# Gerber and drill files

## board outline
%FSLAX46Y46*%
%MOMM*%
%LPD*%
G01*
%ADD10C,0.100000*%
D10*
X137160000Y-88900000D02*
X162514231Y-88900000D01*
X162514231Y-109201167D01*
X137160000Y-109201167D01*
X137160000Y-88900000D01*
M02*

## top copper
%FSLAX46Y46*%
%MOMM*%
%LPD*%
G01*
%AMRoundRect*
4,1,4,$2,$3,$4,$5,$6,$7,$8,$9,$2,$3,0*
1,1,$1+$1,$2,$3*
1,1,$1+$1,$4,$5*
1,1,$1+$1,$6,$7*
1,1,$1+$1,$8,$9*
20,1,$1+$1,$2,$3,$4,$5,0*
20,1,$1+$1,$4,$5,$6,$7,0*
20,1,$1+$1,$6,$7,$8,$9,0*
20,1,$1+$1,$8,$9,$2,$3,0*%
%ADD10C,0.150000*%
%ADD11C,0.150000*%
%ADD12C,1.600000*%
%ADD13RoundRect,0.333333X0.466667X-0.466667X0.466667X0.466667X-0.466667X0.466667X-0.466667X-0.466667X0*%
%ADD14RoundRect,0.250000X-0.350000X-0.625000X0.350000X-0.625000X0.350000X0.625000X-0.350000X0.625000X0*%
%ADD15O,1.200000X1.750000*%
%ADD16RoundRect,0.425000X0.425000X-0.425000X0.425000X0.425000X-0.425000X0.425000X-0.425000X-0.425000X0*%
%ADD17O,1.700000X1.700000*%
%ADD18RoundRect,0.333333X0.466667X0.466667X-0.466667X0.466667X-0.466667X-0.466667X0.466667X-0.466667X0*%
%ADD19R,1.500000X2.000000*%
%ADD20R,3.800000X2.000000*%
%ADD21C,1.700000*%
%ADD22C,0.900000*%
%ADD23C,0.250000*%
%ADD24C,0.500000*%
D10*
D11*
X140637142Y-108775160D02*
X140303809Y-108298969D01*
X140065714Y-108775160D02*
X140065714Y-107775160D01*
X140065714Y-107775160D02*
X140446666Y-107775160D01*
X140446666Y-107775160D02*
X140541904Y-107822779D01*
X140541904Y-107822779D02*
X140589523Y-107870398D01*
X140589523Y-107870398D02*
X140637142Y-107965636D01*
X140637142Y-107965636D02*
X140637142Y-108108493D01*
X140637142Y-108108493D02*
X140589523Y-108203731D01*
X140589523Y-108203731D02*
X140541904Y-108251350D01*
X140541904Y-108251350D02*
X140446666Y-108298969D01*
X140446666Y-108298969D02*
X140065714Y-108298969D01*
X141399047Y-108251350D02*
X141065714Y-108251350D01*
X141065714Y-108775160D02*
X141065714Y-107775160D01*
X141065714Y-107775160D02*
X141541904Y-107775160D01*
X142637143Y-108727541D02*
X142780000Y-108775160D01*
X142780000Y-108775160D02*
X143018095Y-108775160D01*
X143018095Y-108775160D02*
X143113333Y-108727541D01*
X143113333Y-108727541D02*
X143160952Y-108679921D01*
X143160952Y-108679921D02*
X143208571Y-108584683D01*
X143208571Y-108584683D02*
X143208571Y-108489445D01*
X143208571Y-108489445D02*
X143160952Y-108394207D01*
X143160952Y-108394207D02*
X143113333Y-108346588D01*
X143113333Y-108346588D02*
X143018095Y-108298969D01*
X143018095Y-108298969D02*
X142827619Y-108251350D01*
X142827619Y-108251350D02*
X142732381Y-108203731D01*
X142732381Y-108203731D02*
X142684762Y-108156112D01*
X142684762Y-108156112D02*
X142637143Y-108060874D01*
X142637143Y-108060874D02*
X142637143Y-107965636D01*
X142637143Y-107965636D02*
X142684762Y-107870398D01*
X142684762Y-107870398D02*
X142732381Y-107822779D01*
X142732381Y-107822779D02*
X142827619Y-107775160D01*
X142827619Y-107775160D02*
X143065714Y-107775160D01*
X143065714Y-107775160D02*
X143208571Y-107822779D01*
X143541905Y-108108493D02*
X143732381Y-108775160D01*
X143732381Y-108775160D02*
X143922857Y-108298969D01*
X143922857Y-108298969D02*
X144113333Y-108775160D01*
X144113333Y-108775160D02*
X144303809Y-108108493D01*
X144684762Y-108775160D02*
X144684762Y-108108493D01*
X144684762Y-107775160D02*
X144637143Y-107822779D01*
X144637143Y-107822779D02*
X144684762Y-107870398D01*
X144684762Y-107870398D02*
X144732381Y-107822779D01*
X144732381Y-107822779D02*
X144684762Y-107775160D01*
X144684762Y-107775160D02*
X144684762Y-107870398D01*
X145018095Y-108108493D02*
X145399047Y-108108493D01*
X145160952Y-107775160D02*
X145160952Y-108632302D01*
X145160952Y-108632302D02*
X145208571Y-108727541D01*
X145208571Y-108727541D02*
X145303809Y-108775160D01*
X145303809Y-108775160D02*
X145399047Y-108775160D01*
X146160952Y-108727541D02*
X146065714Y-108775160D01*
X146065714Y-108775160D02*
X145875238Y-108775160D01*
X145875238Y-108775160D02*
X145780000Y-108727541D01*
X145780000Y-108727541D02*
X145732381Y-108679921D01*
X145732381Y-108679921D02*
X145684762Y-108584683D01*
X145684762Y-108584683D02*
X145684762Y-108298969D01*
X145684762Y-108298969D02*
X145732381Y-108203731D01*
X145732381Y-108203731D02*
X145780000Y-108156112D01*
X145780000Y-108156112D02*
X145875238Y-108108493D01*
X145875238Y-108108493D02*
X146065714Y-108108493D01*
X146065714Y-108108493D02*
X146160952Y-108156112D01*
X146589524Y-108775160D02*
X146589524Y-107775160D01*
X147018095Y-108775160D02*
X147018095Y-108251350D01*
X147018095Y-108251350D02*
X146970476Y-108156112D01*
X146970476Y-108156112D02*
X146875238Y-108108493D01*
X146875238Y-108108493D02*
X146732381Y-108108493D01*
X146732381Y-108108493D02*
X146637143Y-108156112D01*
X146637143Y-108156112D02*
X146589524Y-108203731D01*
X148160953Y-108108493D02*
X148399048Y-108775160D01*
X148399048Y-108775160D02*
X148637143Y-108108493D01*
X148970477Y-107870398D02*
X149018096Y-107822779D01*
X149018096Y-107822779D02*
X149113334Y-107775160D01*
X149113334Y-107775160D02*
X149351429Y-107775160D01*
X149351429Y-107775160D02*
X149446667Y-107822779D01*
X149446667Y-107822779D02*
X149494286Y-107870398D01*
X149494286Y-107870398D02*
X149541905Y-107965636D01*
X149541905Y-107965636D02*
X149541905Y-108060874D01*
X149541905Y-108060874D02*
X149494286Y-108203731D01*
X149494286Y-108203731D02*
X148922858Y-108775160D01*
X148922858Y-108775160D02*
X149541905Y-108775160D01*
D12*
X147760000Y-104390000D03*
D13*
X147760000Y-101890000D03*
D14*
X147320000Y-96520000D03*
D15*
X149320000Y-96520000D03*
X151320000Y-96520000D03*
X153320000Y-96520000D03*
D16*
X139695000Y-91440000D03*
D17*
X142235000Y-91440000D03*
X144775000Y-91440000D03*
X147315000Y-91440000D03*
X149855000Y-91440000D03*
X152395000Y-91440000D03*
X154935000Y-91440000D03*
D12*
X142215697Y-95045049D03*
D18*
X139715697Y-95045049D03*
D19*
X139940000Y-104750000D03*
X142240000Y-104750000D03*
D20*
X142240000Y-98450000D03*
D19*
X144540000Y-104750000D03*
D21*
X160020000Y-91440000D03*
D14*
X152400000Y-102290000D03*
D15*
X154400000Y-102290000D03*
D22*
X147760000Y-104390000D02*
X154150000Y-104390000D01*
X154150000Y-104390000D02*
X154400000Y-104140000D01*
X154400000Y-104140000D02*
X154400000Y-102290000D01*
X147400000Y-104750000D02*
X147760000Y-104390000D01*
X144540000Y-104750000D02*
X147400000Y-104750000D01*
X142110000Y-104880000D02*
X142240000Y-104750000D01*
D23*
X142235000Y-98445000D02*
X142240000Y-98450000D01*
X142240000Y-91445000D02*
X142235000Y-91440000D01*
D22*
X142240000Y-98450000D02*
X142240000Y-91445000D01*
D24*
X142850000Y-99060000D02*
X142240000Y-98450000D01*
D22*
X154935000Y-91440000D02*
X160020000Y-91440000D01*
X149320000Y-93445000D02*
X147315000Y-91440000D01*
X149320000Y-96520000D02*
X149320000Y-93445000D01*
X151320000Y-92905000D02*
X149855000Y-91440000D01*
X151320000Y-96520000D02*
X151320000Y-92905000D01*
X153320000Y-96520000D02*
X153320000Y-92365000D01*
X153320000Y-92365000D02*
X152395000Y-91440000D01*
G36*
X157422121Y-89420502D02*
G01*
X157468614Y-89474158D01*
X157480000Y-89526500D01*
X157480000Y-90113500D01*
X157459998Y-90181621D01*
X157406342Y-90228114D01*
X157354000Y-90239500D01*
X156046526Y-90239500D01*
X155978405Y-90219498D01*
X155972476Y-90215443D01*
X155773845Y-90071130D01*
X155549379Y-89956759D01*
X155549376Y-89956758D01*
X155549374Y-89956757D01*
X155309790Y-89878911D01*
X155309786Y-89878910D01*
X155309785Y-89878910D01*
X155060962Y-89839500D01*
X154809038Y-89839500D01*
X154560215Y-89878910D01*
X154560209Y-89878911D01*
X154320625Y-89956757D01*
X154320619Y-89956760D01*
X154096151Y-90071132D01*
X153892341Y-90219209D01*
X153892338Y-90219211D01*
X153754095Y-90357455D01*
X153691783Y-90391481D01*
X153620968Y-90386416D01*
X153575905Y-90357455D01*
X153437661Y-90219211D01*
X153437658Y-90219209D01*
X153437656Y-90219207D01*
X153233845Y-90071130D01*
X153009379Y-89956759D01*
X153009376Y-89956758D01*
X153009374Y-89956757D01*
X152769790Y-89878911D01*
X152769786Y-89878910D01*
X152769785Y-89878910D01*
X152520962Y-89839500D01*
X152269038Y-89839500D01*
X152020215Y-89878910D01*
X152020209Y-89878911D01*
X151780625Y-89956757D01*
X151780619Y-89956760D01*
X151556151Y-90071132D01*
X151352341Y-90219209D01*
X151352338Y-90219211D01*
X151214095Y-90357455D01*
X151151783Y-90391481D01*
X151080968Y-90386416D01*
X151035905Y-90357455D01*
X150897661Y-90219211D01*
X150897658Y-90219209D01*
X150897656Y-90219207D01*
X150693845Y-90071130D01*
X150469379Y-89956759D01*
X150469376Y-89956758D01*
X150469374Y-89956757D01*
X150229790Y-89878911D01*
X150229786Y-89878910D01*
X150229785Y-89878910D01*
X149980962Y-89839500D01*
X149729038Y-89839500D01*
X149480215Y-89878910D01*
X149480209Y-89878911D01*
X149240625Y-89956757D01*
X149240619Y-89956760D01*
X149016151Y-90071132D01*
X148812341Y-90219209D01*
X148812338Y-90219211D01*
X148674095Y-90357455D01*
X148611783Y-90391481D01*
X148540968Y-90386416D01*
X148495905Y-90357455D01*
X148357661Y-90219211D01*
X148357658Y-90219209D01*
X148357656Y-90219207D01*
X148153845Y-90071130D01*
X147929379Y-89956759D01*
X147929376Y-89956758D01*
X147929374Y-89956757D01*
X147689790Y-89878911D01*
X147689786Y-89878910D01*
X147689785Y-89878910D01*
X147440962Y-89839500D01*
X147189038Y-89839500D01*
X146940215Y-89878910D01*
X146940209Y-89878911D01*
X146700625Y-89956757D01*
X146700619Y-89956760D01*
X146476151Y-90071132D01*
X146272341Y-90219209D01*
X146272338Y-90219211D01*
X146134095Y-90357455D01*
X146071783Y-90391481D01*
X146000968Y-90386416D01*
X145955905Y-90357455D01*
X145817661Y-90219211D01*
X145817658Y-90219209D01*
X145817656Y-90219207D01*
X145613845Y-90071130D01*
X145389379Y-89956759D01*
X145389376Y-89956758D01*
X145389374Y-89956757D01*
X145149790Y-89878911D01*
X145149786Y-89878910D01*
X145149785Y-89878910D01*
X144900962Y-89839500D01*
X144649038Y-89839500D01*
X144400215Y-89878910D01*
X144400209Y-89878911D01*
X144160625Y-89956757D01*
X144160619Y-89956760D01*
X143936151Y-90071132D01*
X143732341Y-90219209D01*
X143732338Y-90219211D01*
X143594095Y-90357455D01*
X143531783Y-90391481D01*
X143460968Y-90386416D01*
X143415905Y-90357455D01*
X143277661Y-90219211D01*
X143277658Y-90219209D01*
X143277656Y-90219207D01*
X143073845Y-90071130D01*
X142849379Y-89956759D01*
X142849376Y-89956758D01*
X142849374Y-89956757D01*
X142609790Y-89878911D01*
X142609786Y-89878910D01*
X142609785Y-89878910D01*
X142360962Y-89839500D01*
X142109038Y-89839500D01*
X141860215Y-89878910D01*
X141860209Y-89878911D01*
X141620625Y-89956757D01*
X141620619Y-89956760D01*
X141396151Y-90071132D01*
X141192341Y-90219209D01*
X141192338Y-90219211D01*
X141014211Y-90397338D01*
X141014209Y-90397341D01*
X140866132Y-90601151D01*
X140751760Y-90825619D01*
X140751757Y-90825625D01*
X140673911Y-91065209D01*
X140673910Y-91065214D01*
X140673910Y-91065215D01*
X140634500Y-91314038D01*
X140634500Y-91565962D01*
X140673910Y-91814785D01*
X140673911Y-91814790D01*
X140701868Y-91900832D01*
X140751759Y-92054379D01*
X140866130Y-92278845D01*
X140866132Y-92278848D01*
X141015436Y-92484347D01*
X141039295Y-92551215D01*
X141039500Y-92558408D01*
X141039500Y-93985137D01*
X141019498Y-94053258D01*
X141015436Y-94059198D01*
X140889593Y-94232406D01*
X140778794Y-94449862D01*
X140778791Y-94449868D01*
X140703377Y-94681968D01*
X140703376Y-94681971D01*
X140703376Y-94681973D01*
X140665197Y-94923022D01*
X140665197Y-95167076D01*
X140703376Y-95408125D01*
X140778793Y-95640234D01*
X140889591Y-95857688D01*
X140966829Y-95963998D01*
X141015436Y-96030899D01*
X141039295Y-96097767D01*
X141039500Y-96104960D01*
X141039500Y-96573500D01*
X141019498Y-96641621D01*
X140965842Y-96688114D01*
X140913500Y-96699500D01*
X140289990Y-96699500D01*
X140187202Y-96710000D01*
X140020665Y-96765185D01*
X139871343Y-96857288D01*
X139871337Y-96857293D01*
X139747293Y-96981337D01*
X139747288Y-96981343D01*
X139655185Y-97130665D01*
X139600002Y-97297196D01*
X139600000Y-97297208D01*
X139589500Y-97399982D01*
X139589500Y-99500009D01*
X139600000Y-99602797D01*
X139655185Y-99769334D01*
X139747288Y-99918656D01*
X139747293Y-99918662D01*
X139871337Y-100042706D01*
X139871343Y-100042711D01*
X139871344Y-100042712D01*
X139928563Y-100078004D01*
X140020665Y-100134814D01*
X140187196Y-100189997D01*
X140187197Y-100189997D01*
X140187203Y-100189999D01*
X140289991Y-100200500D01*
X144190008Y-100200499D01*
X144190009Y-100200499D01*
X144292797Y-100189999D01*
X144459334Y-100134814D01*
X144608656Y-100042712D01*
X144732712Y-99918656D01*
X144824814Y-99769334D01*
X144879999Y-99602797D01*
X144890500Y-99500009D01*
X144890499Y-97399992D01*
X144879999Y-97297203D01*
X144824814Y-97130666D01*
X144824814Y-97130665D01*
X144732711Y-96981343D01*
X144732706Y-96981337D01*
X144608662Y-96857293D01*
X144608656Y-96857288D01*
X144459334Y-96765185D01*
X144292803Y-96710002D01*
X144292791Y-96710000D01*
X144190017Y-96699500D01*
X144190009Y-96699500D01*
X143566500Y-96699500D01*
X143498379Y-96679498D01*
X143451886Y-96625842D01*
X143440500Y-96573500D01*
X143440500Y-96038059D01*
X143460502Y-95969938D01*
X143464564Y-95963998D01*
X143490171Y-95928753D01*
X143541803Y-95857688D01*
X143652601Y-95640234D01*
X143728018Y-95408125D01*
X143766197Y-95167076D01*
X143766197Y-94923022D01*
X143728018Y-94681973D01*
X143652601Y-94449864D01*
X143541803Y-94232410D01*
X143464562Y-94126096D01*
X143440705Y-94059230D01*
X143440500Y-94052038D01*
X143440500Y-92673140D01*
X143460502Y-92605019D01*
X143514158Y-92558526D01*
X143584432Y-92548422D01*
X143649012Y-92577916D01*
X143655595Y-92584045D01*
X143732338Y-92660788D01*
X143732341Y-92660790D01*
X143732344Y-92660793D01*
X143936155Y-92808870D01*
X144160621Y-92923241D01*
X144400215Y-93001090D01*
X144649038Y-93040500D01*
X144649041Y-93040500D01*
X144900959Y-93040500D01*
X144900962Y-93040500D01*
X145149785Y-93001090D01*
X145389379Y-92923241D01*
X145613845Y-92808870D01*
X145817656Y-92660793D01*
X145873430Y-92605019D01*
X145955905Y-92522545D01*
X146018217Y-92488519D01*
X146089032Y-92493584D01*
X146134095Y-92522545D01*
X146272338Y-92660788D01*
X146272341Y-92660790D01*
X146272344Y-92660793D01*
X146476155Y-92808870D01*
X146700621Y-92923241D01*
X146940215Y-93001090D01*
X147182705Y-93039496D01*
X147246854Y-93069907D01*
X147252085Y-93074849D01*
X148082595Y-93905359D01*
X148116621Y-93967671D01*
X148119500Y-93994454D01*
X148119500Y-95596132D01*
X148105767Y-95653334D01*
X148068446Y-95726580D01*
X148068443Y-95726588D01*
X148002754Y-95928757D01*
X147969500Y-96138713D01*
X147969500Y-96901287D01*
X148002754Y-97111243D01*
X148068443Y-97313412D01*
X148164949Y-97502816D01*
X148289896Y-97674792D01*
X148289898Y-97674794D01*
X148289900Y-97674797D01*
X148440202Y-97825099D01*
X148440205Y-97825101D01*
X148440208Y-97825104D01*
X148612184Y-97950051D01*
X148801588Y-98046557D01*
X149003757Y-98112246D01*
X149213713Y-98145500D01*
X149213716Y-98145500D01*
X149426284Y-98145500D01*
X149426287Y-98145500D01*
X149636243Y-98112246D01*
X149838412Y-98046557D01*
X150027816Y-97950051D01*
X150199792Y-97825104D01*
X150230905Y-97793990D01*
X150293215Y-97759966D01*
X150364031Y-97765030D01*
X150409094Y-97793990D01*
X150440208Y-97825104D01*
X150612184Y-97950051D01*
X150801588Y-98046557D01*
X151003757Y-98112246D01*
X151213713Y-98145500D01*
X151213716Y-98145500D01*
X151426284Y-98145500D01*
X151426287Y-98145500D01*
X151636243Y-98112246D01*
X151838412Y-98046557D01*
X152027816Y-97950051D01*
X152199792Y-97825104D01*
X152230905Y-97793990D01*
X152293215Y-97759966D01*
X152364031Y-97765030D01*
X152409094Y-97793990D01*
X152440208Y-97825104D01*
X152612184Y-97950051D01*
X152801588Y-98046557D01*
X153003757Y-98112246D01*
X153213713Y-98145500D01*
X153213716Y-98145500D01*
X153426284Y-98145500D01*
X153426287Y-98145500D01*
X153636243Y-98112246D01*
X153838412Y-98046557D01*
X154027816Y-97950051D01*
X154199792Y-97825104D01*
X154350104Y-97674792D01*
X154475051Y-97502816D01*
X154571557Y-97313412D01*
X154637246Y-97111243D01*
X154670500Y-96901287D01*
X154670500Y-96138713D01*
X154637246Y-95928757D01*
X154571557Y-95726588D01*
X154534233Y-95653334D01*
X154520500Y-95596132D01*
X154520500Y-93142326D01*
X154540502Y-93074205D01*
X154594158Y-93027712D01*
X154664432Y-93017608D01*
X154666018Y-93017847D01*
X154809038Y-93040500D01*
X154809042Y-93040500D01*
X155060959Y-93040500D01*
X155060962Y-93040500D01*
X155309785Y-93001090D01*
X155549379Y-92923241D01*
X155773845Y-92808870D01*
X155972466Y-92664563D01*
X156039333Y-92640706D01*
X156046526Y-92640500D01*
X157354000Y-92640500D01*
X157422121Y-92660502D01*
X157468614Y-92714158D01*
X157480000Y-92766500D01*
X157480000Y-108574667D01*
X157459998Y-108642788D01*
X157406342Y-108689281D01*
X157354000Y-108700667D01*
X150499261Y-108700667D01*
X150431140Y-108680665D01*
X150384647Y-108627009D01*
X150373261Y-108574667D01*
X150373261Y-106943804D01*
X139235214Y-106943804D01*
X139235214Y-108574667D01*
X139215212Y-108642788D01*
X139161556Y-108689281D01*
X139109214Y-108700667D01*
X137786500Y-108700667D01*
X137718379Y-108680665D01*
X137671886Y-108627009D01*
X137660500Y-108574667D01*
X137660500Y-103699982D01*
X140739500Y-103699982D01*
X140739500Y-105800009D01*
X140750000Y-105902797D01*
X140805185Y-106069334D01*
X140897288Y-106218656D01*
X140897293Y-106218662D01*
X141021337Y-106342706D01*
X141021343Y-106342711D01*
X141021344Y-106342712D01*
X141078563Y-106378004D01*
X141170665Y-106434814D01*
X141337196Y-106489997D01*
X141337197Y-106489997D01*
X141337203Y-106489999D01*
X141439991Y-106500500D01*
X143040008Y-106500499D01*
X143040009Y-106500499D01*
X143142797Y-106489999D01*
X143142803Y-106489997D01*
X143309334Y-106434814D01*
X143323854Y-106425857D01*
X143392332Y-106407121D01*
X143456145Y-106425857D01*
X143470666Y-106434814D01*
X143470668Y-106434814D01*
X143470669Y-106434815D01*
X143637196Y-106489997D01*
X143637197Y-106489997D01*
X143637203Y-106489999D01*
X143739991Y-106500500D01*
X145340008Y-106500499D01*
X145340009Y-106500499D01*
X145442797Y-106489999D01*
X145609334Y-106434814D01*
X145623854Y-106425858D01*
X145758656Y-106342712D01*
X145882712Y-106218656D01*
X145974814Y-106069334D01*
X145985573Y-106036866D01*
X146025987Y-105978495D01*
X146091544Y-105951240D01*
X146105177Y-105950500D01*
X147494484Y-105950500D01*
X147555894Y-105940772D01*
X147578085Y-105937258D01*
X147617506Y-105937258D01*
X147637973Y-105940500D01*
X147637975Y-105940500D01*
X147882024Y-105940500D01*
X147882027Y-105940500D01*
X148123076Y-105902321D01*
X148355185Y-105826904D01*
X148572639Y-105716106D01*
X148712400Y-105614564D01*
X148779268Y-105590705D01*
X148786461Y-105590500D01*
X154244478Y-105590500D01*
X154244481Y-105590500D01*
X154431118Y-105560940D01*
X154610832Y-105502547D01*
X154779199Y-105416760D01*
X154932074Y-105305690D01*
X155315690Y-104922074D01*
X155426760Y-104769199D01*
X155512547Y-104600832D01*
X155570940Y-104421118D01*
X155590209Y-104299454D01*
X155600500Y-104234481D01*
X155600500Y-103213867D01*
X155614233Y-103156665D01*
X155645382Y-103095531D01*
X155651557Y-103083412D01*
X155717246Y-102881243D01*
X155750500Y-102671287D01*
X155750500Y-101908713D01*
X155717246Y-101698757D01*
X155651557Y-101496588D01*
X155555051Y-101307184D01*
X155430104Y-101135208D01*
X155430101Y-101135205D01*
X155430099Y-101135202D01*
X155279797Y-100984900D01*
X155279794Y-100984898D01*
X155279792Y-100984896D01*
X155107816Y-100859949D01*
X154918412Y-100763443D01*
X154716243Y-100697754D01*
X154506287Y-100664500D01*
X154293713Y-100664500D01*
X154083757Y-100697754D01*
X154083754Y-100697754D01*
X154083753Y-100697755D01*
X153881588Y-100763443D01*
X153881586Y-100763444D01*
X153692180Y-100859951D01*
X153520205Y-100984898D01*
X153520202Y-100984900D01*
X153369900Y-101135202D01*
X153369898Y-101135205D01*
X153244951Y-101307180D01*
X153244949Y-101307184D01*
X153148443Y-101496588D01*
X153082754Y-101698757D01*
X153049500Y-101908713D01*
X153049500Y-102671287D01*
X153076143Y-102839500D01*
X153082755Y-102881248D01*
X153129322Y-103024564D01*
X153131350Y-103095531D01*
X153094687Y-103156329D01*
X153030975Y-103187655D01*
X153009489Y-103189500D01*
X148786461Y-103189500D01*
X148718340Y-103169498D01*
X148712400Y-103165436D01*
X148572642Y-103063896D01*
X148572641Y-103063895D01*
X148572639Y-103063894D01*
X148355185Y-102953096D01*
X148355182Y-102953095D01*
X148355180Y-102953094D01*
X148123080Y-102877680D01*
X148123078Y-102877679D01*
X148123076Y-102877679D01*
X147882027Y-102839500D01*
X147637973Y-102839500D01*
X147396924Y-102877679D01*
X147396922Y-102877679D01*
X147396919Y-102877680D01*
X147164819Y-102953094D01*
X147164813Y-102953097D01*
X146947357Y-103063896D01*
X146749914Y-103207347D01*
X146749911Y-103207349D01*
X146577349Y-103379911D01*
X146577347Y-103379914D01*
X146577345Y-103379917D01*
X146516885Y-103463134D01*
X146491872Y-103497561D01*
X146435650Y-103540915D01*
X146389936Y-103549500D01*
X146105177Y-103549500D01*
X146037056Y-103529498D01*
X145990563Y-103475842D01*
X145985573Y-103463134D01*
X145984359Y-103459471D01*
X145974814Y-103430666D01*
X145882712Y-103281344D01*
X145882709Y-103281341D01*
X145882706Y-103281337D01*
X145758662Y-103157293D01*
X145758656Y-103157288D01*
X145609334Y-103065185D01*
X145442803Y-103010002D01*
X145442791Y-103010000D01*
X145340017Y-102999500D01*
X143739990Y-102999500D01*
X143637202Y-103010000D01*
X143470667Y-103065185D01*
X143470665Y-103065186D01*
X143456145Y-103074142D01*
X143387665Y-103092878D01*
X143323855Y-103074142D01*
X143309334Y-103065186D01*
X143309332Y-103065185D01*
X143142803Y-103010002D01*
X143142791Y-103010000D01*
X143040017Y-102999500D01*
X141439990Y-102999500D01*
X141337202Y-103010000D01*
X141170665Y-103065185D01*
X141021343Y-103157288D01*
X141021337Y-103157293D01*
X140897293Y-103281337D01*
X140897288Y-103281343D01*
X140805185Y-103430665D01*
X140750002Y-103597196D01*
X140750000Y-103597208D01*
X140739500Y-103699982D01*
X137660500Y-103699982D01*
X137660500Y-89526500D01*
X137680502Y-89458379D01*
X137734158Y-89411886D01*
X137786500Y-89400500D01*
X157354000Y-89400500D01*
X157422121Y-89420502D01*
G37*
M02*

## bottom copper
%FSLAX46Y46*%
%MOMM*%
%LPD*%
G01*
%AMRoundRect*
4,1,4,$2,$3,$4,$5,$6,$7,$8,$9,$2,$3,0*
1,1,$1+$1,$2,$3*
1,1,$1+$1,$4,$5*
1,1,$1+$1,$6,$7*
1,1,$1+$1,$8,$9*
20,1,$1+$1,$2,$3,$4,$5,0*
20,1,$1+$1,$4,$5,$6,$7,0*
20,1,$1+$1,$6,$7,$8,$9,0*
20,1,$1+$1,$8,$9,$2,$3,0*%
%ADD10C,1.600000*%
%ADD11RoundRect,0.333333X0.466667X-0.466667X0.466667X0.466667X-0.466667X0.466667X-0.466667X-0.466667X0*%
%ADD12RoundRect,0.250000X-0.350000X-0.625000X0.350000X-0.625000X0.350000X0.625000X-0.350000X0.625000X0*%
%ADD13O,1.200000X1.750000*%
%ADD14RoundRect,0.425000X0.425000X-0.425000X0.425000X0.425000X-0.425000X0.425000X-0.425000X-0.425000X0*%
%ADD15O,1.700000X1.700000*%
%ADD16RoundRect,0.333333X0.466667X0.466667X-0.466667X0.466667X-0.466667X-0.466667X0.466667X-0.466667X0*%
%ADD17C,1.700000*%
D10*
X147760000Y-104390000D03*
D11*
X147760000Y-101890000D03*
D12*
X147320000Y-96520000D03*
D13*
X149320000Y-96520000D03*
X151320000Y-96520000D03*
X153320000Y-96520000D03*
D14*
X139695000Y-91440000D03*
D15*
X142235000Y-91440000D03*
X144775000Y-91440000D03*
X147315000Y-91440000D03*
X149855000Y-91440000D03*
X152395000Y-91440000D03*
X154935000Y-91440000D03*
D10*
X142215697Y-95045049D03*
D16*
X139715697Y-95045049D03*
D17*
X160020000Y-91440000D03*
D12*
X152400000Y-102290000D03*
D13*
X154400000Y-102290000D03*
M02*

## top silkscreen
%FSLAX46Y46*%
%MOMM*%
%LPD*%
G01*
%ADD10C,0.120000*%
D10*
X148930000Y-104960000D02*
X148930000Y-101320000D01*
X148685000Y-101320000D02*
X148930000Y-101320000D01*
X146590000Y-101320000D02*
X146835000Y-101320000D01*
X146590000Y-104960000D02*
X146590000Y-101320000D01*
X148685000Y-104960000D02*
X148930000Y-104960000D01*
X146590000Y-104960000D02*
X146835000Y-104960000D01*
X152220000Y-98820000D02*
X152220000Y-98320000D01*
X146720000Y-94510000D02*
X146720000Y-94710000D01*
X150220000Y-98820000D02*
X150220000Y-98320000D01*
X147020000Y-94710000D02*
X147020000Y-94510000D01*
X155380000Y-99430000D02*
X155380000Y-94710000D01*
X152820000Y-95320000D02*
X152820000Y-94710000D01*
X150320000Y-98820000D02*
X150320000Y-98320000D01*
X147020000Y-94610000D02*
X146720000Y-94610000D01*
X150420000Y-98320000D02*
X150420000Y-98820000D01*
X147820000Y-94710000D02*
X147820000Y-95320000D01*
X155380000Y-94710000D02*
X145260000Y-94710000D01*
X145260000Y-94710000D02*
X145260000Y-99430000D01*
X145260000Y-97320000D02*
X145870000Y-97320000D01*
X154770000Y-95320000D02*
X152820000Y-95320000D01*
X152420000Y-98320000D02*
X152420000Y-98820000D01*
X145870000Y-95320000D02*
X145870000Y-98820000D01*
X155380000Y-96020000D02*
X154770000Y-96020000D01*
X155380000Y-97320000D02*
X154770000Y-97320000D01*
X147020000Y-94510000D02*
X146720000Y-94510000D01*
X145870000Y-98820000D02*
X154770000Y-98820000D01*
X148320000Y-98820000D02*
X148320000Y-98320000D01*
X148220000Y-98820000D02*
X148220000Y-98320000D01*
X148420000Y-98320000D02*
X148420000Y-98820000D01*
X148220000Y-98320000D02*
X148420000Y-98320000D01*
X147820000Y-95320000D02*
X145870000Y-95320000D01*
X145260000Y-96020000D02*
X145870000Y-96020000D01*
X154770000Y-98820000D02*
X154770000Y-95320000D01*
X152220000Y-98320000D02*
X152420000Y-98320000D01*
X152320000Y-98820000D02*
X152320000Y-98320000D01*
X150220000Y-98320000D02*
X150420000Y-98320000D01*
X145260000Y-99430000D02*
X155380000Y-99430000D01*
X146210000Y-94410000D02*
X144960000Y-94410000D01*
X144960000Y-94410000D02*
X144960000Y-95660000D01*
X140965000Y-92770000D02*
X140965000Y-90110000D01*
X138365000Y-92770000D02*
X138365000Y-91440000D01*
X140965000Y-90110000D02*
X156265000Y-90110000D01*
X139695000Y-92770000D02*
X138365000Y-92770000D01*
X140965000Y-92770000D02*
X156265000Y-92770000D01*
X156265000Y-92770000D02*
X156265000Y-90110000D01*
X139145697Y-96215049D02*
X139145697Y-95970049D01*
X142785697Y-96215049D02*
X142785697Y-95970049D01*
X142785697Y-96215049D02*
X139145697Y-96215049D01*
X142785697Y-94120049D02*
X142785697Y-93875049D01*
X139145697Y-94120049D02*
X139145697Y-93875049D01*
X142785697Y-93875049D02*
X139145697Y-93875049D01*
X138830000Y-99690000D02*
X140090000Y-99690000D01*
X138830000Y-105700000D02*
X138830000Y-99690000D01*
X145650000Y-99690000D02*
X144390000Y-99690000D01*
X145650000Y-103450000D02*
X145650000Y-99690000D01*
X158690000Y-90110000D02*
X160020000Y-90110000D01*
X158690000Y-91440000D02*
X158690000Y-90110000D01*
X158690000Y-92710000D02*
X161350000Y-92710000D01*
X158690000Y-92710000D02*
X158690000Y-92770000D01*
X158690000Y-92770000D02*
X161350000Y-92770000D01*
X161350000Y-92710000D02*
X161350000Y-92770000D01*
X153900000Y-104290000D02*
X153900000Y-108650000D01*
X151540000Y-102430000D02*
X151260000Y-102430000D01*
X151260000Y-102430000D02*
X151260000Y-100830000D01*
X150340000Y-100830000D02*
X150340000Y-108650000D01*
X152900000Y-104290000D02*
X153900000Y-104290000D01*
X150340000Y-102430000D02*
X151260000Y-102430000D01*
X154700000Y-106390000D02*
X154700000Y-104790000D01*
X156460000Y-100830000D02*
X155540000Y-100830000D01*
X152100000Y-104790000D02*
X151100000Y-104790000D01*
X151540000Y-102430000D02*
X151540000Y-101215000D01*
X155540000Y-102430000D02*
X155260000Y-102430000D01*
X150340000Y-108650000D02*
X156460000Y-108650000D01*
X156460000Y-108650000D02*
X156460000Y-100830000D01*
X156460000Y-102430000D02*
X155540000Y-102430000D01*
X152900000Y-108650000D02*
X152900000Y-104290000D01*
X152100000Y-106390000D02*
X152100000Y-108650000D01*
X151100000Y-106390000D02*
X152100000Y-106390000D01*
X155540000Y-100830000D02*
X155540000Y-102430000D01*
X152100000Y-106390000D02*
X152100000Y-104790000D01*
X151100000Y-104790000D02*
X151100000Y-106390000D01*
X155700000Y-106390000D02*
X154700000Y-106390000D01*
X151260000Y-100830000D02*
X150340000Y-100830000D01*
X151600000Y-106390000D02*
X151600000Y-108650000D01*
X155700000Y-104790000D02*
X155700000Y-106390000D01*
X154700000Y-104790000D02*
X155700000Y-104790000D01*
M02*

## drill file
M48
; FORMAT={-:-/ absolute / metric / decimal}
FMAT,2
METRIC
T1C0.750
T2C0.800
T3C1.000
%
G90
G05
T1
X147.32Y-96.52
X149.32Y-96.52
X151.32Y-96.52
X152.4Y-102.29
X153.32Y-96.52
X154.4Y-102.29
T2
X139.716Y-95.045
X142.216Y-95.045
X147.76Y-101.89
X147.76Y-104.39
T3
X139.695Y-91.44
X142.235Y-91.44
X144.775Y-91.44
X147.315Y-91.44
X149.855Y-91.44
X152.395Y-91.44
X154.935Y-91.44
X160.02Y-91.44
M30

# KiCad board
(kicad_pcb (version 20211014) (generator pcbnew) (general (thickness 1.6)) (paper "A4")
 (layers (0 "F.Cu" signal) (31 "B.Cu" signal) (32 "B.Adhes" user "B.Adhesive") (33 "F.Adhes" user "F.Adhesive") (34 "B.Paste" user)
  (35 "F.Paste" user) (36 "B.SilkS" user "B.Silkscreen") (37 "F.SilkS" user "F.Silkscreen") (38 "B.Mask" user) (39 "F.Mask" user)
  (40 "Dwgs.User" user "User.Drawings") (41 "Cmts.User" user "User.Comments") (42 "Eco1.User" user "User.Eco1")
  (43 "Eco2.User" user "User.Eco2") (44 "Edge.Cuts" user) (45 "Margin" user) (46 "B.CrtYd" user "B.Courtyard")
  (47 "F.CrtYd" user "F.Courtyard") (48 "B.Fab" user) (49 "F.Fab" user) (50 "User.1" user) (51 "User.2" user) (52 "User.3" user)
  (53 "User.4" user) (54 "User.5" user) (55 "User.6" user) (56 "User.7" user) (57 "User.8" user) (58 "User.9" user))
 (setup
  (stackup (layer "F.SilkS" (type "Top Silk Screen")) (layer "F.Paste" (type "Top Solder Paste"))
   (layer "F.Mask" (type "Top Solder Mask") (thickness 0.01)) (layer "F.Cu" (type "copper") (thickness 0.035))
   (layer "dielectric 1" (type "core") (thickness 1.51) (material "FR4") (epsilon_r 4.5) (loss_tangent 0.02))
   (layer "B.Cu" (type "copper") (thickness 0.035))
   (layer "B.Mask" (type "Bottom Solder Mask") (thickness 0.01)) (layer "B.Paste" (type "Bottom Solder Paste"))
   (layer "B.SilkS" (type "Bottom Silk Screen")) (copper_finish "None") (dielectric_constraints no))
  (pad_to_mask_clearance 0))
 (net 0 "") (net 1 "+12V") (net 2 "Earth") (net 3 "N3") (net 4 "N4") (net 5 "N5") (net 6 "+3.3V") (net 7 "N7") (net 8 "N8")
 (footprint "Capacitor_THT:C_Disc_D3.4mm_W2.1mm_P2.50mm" (layer "F.Cu") (at 147.76 104.39 90)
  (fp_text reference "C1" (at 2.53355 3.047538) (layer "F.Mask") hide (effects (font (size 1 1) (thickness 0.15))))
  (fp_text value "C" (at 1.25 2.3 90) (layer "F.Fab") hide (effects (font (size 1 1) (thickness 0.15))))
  (fp_line (start -0.57 1.17) (end 3.07 1.17) (layer "F.SilkS") (width 0.12))
  (fp_line (start 3.07 0.925) (end 3.07 1.17) (layer "F.SilkS") (width 0.12))
  (fp_line (start 3.07 -1.17) (end 3.07 -0.925) (layer "F.SilkS") (width 0.12))
  (fp_line (start -0.57 -1.17) (end 3.07 -1.17) (layer "F.SilkS") (width 0.12))
  (fp_line (start -0.57 0.925) (end -0.57 1.17) (layer "F.SilkS") (width 0.12))
  (fp_line (start -0.57 -1.17) (end -0.57 -0.925) (layer "F.SilkS") (width 0.12))
  (pad "1" thru_hole circle (at 0 0 90) (size 1.6 1.6) (drill 0.8) (layers *.Cu *.Mask) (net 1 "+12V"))
  (pad "2" thru_hole roundrect (at 2.5 0 90) (size 1.6 1.6) (drill 0.8) (layers *.Cu *.Mask) (roundrect_rratio 0.208333) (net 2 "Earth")))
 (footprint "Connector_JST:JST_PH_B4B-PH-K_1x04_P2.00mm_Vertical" (layer "F.Cu") (at 147.32 96.52)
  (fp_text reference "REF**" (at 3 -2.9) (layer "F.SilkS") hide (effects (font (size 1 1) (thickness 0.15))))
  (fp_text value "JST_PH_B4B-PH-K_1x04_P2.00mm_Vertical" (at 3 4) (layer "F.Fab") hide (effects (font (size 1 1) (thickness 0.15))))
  (fp_line (start 4.9 2.3) (end 4.9 1.8) (layer "F.SilkS") (width 0.12))
  (fp_line (start -0.6 -2.01) (end -0.6 -1.81) (layer "F.SilkS") (width 0.12))
  (fp_line (start 2.9 2.3) (end 2.9 1.8) (layer "F.SilkS") (width 0.12))
  (fp_line (start -0.3 -1.81) (end -0.3 -2.01) (layer "F.SilkS") (width 0.12))
  (fp_line (start 8.06 2.91) (end 8.06 -1.81) (layer "F.SilkS") (width 0.12))
  (fp_line (start 5.5 -1.2) (end 5.5 -1.81) (layer "F.SilkS") (width 0.12))
  (fp_line (start 3 2.3) (end 3 1.8) (layer "F.SilkS") (width 0.12))
  (fp_line (start -0.3 -1.91) (end -0.6 -1.91) (layer "F.SilkS") (width 0.12))
  (fp_line (start 3.1 1.8) (end 3.1 2.3) (layer "F.SilkS") (width 0.12))
  (fp_line (start 0.5 -1.81) (end 0.5 -1.2) (layer "F.SilkS") (width 0.12))
  (fp_line (start 8.06 -1.81) (end -2.06 -1.81) (layer "F.SilkS") (width 0.12))
  (fp_line (start -2.06 -1.81) (end -2.06 2.91) (layer "F.SilkS") (width 0.12))
  (fp_line (start -2.06 0.8) (end -1.45 0.8) (layer "F.SilkS") (width 0.12))
  (fp_line (start 7.45 -1.2) (end 5.5 -1.2) (layer "F.SilkS") (width 0.12))
  (fp_line (start 5.1 1.8) (end 5.1 2.3) (layer "F.SilkS") (width 0.12))
  (fp_line (start -1.45 -1.2) (end -1.45 2.3) (layer "F.SilkS") (width 0.12))
  (fp_line (start 8.06 -0.5) (end 7.45 -0.5) (layer "F.SilkS") (width 0.12))
  (fp_line (start 8.06 0.8) (end 7.45 0.8) (layer "F.SilkS") (width 0.12))
  (fp_line (start -0.3 -2.01) (end -0.6 -2.01) (layer "F.SilkS") (width 0.12))
  (fp_line (start -1.45 2.3) (end 7.45 2.3) (layer "F.SilkS") (width 0.12))
  (fp_line (start 1 2.3) (end 1 1.8) (layer "F.SilkS") (width 0.12))
  (fp_line (start 0.9 2.3) (end 0.9 1.8) (layer "F.SilkS") (width 0.12))
  (fp_line (start 1.1 1.8) (end 1.1 2.3) (layer "F.SilkS") (width 0.12))
  (fp_line (start 0.9 1.8) (end 1.1 1.8) (layer "F.SilkS") (width 0.12))
  (fp_line (start 0.5 -1.2) (end -1.45 -1.2) (layer "F.SilkS") (width 0.12))
  (fp_line (start -2.06 -0.5) (end -1.45 -0.5) (layer "F.SilkS") (width 0.12))
  (fp_line (start 7.45 2.3) (end 7.45 -1.2) (layer "F.SilkS") (width 0.12))
  (fp_line (start 4.9 1.8) (end 5.1 1.8) (layer "F.SilkS") (width 0.12))
  (fp_line (start 5 2.3) (end 5 1.8) (layer "F.SilkS") (width 0.12))
  (fp_line (start 2.9 1.8) (end 3.1 1.8) (layer "F.SilkS") (width 0.12))
  (fp_line (start -2.06 2.91) (end 8.06 2.91) (layer "F.SilkS") (width 0.12))
  (fp_line (start -1.11 -2.11) (end -2.36 -2.11) (layer "F.SilkS") (width 0.12))
  (fp_line (start -2.36 -2.11) (end -2.36 -0.86) (layer "F.SilkS") (width 0.12))
  (pad "1" thru_hole roundrect (at 0 0) (size 1.2 1.75) (drill 0.75) (layers *.Cu *.Mask) (roundrect_rratio 0.208333) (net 2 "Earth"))
  (pad "2" thru_hole oval (at 2 0) (size 1.2 1.75) (drill 0.75) (layers *.Cu *.Mask) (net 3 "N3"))
  (pad "3" thru_hole oval (at 4 0) (size 1.2 1.75) (drill 0.75) (layers *.Cu *.Mask) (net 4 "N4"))
  (pad "4" thru_hole oval (at 6 0) (size 1.2 1.75) (drill 0.75) (layers *.Cu *.Mask) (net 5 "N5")))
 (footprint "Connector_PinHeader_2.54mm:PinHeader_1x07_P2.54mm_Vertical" (layer "F.Cu") (at 139.695 91.44 90)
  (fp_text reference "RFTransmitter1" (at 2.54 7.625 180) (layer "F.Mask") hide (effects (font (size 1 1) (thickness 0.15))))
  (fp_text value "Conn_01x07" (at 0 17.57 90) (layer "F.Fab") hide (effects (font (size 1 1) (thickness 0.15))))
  (fp_line (start -1.33 1.27) (end 1.33 1.27) (layer "F.SilkS") (width 0.12))
  (fp_line (start -1.33 -1.33) (end 0 -1.33) (layer "F.SilkS") (width 0.12))
  (fp_line (start 1.33 1.27) (end 1.33 16.57) (layer "F.SilkS") (width 0.12))
  (fp_line (start -1.33 0) (end -1.33 -1.33) (layer "F.SilkS") (width 0.12))
  (fp_line (start -1.33 1.27) (end -1.33 16.57) (layer "F.SilkS") (width 0.12))
  (fp_line (start -1.33 16.57) (end 1.33 16.57) (layer "F.SilkS") (width 0.12))
  (pad "1" thru_hole roundrect (at 0 0 90) (size 1.7 1.7) (drill 1) (layers *.Cu *.Mask) (roundrect_rratio 0.25) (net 2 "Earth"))
  (pad "2" thru_hole oval (at 0 2.54 90) (size 1.7 1.7) (drill 1) (layers *.Cu *.Mask) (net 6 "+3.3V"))
  (pad "3" thru_hole oval (at 0 5.08 90) (size 1.7 1.7) (drill 1) (layers *.Cu *.Mask) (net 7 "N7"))
  (pad "4" thru_hole oval (at 0 7.62 90) (size 1.7 1.7) (drill 1) (layers *.Cu *.Mask) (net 3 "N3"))
  (pad "5" thru_hole oval (at 0 10.16 90) (size 1.7 1.7) (drill 1) (layers *.Cu *.Mask) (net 4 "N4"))
  (pad "6" thru_hole oval (at 0 12.7 90) (size 1.7 1.7) (drill 1) (layers *.Cu *.Mask) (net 5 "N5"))
  (pad "7" thru_hole oval (at 0 15.24 90) (size 1.7 1.7) (drill 1) (layers *.Cu *.Mask) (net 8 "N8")))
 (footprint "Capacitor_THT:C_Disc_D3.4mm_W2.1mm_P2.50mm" (layer "F.Cu") (at 142.215697 95.045049 180)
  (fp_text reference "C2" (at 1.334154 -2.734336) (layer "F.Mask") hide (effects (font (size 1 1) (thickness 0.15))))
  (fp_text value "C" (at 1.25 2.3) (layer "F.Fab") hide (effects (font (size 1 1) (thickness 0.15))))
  (fp_line (start 3.07 -1.17) (end 3.07 -0.925) (layer "F.SilkS") (width 0.12))
  (fp_line (start -0.57 -1.17) (end -0.57 -0.925) (layer "F.SilkS") (width 0.12))
  (fp_line (start -0.57 -1.17) (end 3.07 -1.17) (layer "F.SilkS") (width 0.12))
  (fp_line (start -0.57 0.925) (end -0.57 1.17) (layer "F.SilkS") (width 0.12))
  (fp_line (start 3.07 0.925) (end 3.07 1.17) (layer "F.SilkS") (width 0.12))
  (fp_line (start -0.57 1.17) (end 3.07 1.17) (layer "F.SilkS") (width 0.12))
  (pad "1" thru_hole circle (at 0 0 180) (size 1.6 1.6) (drill 0.8) (layers *.Cu *.Mask) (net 6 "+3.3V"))
  (pad "2" thru_hole roundrect (at 2.5 0 180) (size 1.6 1.6) (drill 0.8) (layers *.Cu *.Mask) (roundrect_rratio 0.208333) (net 2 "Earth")))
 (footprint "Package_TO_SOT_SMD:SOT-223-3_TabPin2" (layer "F.Cu") (at 142.24 101.6 90)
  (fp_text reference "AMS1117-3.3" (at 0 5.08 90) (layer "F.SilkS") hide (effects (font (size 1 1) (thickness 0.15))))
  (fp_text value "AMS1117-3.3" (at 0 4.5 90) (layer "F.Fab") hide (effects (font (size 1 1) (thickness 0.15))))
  (fp_line (start 1.91 -3.41) (end 1.91 -2.15) (layer "F.SilkS") (width 0.12))
  (fp_line (start -4.1 -3.41) (end 1.91 -3.41) (layer "F.SilkS") (width 0.12))
  (fp_line (start 1.91 3.41) (end 1.91 2.15) (layer "F.SilkS") (width 0.12))
  (fp_line (start -1.85 3.41) (end 1.91 3.41) (layer "F.SilkS") (width 0.12))
  (pad "1" smd rect (at -3.15 -2.3 90) (size 2 1.5) (layers "F.Cu" "F.Paste" "F.Mask") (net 2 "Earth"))
  (pad "2" smd rect (at -3.15 0 90) (size 2 1.5) (layers "F.Cu" "F.Paste" "F.Mask") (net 6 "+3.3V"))
  (pad "2" smd rect (at 3.15 0 90) (size 2 3.8) (layers "F.Cu" "F.Paste" "F.Mask") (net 6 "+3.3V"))
  (pad "3" smd rect (at -3.15 2.3 90) (size 2 1.5) (layers "F.Cu" "F.Paste" "F.Mask") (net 1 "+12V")))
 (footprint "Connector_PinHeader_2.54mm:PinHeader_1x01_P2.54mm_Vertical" (layer "F.Cu") (at 160.02 91.44)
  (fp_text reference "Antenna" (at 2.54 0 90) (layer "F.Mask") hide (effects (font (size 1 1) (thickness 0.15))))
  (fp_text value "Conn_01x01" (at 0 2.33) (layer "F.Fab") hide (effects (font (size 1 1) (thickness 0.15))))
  (fp_line (start -1.33 -1.33) (end 0 -1.33) (layer "F.SilkS") (width 0.12))
  (fp_line (start -1.33 0) (end -1.33 -1.33) (layer "F.SilkS") (width 0.12))
  (fp_line (start -1.33 1.27) (end 1.33 1.27) (layer "F.SilkS") (width 0.12))
  (fp_line (start -1.33 1.27) (end -1.33 1.33) (layer "F.SilkS") (width 0.12))
  (fp_line (start -1.33 1.33) (end 1.33 1.33) (layer "F.SilkS") (width 0.12))
  (fp_line (start 1.33 1.27) (end 1.33 1.33) (layer "F.SilkS") (width 0.12))
  (pad "1" thru_hole circle (at 0 0) (size 1.7 1.7) (drill 1) (layers *.Cu *.Mask) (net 8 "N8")))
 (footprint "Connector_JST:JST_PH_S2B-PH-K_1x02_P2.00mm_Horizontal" (layer "F.Cu") (at 152.4 102.29)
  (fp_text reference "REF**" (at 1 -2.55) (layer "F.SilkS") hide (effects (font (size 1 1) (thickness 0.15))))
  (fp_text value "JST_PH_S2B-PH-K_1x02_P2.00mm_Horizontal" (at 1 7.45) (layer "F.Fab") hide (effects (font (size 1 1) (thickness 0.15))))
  (fp_line (start 1.5 2) (end 1.5 6.36) (layer "F.SilkS") (width 0.12))
  (fp_line (start -0.86 0.14) (end -1.14 0.14) (layer "F.SilkS") (width 0.12))
  (fp_line (start -1.14 0.14) (end -1.14 -1.46) (layer "F.SilkS") (width 0.12))
  (fp_line (start -2.06 -1.46) (end -2.06 6.36) (layer "F.SilkS") (width 0.12))
  (fp_line (start 0.5 2) (end 1.5 2) (layer "F.SilkS") (width 0.12))
  (fp_line (start -2.06 0.14) (end -1.14 0.14) (layer "F.SilkS") (width 0.12))
  (fp_line (start 2.3 4.1) (end 2.3 2.5) (layer "F.SilkS") (width 0.12))
  (fp_line (start 4.06 -1.46) (end 3.14 -1.46) (layer "F.SilkS") (width 0.12))
  (fp_line (start -0.3 2.5) (end -1.3 2.5) (layer "F.SilkS") (width 0.12))
  (fp_line (start -0.86 0.14) (end -0.86 -1.075) (layer "F.SilkS") (width 0.12))
  (fp_line (start 3.14 0.14) (end 2.86 0.14) (layer "F.SilkS") (width 0.12))
  (fp_line (start -2.06 6.36) (end 4.06 6.36) (layer "F.SilkS") (width 0.12))
  (fp_line (start 4.06 6.36) (end 4.06 -1.46) (layer "F.SilkS") (width 0.12))
  (fp_line (start 4.06 0.14) (end 3.14 0.14) (layer "F.SilkS") (width 0.12))
  (fp_line (start 0.5 6.36) (end 0.5 2) (layer "F.SilkS") (width 0.12))
  (fp_line (start -0.3 4.1) (end -0.3 6.36) (layer "F.SilkS") (width 0.12))
  (fp_line (start -1.3 4.1) (end -0.3 4.1) (layer "F.SilkS") (width 0.12))
  (fp_line (start 3.14 -1.46) (end 3.14 0.14) (layer "F.SilkS") (width 0.12))
  (fp_line (start -0.3 4.1) (end -0.3 2.5) (layer "F.SilkS") (width 0.12))
  (fp_line (start -1.3 2.5) (end -1.3 4.1) (layer "F.SilkS") (width 0.12))
  (fp_line (start 3.3 4.1) (end 2.3 4.1) (layer "F.SilkS") (width 0.12))
  (fp_line (start -1.14 -1.46) (end -2.06 -1.46) (layer "F.SilkS") (width 0.12))
  (fp_line (start -0.8 4.1) (end -0.8 6.36) (layer "F.SilkS") (width 0.12))
  (fp_line (start 3.3 2.5) (end 3.3 4.1) (layer "F.SilkS") (width 0.12))
  (fp_line (start 2.3 2.5) (end 3.3 2.5) (layer "F.SilkS") (width 0.12))
  (pad "1" thru_hole roundrect (at 0 0) (size 1.2 1.75) (drill 0.75) (layers *.Cu *.Mask) (roundrect_rratio 0.208333) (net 2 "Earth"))
  (pad "2" thru_hole oval (at 2 0) (size 1.2 1.75) (drill 0.75) (layers *.Cu *.Mask) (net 1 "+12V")))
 (gr_rect (start 137.16 88.9) (end 162.514231 109.201167) (layer "Edge.Cuts") (width 0.1) (fill none))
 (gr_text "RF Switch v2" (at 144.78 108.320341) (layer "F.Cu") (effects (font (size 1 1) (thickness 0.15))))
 (segment (start 147.76 104.39) (end 154.15 104.39) (width 0.9) (layer "F.Cu") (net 1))
 (segment (start 154.15 104.39) (end 154.4 104.14) (width 0.9) (layer "F.Cu") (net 1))
 (segment (start 154.4 104.14) (end 154.4 102.29) (width 0.9) (layer "F.Cu") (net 1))
 (segment (start 147.4 104.75) (end 147.76 104.39) (width 0.9) (layer "F.Cu") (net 1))
 (segment (start 144.54 104.75) (end 147.4 104.75) (width 0.9) (layer "F.Cu") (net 1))
 (segment (start 142.11 104.88) (end 142.24 104.75) (width 0.9) (layer "F.Cu") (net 6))
 (segment (start 142.235 98.445) (end 142.24 98.45) (width 0.25) (layer "F.Cu") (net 6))
 (segment (start 142.24 91.445) (end 142.235 91.44) (width 0.25) (layer "F.Cu") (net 6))
 (segment (start 142.24 98.45) (end 142.24 91.445) (width 0.9) (layer "F.Cu") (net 6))
 (segment (start 142.85 99.06) (end 142.24 98.45) (width 0.5) (layer "F.Cu") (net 6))
 (segment (start 154.935 91.44) (end 160.02 91.44) (width 0.9) (layer "F.Cu") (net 8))
 (segment (start 149.32 93.445) (end 147.315 91.44) (width 0.9) (layer "F.Cu") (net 3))
 (segment (start 149.32 96.52) (end 149.32 93.445) (width 0.9) (layer "F.Cu") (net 3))
 (segment (start 151.32 92.905) (end 149.855 91.44) (width 0.9) (layer "F.Cu") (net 4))
 (segment (start 151.32 96.52) (end 151.32 92.905) (width 0.9) (layer "F.Cu") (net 4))
 (segment (start 153.32 96.52) (end 153.32 92.365) (width 0.9) (layer "F.Cu") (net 5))
 (segment (start 153.32 92.365) (end 152.395 91.44) (width 0.9) (layer "F.Cu") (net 5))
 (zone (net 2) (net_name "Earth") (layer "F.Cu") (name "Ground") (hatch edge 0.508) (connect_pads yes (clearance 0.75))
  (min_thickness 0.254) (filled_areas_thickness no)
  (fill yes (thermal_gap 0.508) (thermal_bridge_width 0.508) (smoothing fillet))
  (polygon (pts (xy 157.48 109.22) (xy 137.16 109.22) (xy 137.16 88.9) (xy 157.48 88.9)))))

